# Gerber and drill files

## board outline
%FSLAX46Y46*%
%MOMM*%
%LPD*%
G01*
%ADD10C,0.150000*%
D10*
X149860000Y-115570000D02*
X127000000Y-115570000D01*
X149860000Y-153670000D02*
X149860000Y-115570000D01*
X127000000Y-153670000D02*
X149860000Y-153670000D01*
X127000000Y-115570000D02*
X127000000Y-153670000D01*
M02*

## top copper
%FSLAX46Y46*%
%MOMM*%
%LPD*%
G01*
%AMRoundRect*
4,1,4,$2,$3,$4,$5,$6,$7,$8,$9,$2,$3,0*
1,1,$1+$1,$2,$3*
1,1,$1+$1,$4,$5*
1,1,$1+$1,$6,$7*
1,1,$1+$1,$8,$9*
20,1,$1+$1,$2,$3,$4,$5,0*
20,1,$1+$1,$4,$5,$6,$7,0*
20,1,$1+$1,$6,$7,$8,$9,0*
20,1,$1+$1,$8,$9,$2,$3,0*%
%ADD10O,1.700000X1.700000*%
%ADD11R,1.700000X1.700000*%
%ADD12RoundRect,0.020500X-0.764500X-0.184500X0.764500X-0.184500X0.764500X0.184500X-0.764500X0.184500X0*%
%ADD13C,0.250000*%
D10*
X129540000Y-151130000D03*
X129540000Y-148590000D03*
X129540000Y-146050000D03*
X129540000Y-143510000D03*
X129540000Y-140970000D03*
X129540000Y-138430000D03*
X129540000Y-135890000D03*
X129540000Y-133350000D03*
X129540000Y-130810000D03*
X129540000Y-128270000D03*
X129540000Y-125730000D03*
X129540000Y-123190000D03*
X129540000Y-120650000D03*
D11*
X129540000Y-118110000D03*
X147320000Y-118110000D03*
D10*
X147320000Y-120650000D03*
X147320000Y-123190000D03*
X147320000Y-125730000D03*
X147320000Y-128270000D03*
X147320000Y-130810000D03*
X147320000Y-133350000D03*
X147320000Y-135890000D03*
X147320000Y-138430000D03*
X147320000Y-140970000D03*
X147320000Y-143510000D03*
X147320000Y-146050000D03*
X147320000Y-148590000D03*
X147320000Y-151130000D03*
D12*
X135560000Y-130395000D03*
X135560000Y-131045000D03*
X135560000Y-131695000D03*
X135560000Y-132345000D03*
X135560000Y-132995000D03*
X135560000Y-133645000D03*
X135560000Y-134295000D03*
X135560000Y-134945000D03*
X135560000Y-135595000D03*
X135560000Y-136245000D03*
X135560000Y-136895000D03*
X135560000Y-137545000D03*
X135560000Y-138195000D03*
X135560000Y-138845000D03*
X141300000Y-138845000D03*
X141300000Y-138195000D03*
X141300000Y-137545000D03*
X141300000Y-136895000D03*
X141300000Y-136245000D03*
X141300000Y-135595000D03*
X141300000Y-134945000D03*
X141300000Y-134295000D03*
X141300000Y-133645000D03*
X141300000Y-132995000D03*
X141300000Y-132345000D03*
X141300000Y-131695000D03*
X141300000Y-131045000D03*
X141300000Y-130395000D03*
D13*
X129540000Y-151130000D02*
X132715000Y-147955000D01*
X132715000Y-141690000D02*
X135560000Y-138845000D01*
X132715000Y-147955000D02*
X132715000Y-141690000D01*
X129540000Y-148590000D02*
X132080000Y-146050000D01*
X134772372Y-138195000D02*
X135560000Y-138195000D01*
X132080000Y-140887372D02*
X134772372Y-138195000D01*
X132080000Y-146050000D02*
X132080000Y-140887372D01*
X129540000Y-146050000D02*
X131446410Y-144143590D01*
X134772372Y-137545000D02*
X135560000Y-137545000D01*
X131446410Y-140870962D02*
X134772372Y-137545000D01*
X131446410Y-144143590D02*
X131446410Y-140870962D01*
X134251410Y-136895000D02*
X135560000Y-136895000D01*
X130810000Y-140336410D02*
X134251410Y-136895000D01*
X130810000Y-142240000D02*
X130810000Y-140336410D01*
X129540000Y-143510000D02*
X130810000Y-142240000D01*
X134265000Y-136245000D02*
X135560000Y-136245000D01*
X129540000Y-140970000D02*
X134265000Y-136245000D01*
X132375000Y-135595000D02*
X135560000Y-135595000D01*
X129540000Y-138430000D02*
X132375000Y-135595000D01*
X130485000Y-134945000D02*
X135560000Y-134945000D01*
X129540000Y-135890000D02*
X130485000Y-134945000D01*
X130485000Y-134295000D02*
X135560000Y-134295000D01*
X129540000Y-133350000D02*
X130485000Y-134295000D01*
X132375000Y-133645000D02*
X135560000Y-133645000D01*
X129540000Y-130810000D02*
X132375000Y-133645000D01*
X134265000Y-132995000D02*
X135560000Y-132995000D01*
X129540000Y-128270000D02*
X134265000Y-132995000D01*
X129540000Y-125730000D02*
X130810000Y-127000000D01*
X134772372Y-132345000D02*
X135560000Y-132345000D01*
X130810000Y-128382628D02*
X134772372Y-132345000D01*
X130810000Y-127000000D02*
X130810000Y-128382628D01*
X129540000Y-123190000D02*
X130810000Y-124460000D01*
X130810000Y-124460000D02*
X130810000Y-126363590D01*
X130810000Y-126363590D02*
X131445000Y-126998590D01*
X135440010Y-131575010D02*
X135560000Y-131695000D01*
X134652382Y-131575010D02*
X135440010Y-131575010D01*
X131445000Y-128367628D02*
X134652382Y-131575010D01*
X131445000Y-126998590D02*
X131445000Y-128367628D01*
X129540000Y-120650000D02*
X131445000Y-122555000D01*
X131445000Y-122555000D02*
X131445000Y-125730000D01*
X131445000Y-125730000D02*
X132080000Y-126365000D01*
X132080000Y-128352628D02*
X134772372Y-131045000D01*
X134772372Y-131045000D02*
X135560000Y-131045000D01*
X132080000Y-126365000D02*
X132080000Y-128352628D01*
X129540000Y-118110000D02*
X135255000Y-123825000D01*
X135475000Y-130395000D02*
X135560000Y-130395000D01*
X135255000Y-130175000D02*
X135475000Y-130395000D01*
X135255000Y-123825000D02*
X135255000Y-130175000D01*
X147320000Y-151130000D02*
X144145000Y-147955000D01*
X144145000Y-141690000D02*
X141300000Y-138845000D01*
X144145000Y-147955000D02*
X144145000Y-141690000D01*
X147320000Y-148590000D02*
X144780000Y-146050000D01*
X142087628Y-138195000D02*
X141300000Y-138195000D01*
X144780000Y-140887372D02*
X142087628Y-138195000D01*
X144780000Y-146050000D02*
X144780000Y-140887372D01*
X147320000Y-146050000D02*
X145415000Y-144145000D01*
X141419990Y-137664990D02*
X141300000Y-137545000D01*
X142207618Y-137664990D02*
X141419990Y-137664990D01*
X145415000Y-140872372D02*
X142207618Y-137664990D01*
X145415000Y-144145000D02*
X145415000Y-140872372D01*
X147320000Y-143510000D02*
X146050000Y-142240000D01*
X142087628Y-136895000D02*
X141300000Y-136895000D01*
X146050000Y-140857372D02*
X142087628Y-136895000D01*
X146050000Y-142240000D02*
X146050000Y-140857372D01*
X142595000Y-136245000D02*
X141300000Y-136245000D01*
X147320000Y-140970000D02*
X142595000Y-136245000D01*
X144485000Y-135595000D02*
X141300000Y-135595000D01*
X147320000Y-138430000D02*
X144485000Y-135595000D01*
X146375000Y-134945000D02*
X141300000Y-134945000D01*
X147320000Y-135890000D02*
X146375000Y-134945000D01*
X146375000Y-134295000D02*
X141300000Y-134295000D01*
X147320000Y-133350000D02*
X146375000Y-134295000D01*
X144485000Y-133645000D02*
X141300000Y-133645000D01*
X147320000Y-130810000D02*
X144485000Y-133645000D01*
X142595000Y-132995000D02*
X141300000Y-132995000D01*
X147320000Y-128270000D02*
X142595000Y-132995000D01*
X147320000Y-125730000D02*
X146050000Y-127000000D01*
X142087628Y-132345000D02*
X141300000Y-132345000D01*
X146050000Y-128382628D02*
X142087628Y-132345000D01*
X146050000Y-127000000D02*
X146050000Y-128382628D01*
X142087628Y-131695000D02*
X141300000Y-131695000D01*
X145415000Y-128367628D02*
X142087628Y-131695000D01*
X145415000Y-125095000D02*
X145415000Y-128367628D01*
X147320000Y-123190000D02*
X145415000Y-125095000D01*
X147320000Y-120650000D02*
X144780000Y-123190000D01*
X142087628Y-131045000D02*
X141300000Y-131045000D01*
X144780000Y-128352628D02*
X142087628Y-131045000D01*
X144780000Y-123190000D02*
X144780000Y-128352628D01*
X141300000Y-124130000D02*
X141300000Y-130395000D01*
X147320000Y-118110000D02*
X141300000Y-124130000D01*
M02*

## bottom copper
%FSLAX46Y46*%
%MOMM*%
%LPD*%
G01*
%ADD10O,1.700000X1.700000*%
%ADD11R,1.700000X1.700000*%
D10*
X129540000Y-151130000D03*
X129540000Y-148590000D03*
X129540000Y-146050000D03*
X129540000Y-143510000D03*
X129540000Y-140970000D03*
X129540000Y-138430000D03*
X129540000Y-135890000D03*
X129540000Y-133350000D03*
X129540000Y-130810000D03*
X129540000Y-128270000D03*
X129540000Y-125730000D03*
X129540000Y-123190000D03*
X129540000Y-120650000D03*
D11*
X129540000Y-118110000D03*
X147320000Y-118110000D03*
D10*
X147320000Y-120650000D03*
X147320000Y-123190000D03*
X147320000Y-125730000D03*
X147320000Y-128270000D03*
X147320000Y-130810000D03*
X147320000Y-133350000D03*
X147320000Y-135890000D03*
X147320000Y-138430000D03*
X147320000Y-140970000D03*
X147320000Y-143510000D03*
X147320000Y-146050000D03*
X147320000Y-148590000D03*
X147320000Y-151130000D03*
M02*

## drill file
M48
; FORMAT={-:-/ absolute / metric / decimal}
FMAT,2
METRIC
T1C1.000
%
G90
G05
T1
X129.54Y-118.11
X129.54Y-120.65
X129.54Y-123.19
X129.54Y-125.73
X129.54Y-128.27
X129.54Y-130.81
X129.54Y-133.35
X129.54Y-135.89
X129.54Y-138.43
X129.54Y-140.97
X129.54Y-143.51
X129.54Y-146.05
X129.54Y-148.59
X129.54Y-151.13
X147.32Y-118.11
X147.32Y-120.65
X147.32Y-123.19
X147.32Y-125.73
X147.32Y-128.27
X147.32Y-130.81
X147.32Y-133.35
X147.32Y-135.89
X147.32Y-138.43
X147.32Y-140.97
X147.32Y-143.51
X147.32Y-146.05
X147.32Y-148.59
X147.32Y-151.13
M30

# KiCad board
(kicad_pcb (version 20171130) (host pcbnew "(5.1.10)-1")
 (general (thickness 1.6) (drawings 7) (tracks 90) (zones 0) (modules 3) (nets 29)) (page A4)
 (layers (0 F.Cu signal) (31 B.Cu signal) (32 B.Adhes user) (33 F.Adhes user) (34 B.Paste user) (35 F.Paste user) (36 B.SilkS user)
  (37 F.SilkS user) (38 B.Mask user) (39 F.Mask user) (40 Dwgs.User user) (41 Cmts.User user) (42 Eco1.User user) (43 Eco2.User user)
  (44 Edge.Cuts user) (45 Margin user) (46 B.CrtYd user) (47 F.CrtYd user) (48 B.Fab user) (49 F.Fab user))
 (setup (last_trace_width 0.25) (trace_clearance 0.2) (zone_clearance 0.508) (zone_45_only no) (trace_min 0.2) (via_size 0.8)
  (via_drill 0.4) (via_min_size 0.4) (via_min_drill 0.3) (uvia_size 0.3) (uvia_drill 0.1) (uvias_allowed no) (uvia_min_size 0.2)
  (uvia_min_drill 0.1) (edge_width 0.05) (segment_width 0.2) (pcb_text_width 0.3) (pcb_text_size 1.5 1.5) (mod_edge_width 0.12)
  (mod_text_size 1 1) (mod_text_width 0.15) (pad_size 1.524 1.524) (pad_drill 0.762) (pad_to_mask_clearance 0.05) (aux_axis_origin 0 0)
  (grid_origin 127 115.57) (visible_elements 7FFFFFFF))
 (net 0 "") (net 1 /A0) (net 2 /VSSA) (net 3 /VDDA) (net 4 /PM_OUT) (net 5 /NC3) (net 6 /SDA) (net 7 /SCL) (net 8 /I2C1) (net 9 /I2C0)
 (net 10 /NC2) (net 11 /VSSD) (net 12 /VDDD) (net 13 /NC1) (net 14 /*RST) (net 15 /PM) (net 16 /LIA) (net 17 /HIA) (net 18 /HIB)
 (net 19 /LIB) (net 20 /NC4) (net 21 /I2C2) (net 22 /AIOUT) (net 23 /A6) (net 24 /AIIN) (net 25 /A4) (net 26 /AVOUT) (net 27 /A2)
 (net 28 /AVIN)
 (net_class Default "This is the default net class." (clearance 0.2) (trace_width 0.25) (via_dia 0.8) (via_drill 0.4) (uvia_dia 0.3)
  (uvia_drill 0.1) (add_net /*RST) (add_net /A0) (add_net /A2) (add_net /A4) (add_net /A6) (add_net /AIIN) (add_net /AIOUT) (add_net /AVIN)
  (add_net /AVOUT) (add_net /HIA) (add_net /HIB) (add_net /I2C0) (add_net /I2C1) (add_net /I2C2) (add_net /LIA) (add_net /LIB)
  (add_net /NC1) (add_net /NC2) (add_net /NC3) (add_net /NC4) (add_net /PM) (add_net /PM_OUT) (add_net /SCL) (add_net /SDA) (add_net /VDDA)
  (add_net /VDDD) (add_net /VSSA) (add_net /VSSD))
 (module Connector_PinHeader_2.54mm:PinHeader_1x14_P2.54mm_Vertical (layer F.Cu) (at 129.54 118.11)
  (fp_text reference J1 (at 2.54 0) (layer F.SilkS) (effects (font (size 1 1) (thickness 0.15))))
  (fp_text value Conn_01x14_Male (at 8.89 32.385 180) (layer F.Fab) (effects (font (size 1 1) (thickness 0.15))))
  (pad 14 thru_hole oval (at 0 33.02) (size 1.7 1.7) (drill 1) (layers *.Cu *.Mask) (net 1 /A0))
  (pad 13 thru_hole oval (at 0 30.48) (size 1.7 1.7) (drill 1) (layers *.Cu *.Mask) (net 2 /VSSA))
  (pad 12 thru_hole oval (at 0 27.94) (size 1.7 1.7) (drill 1) (layers *.Cu *.Mask) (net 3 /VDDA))
  (pad 11 thru_hole oval (at 0 25.4) (size 1.7 1.7) (drill 1) (layers *.Cu *.Mask) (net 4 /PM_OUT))
  (pad 10 thru_hole oval (at 0 22.86) (size 1.7 1.7) (drill 1) (layers *.Cu *.Mask) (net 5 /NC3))
  (pad 9 thru_hole oval (at 0 20.32) (size 1.7 1.7) (drill 1) (layers *.Cu *.Mask) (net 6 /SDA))
  (pad 8 thru_hole oval (at 0 17.78) (size 1.7 1.7) (drill 1) (layers *.Cu *.Mask) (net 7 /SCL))
  (pad 7 thru_hole oval (at 0 15.24) (size 1.7 1.7) (drill 1) (layers *.Cu *.Mask) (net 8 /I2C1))
  (pad 6 thru_hole oval (at 0 12.7) (size 1.7 1.7) (drill 1) (layers *.Cu *.Mask) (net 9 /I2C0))
  (pad 5 thru_hole oval (at 0 10.16) (size 1.7 1.7) (drill 1) (layers *.Cu *.Mask) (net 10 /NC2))
  (pad 4 thru_hole oval (at 0 7.62) (size 1.7 1.7) (drill 1) (layers *.Cu *.Mask) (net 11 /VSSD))
  (pad 3 thru_hole oval (at 0 5.08) (size 1.7 1.7) (drill 1) (layers *.Cu *.Mask) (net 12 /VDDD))
  (pad 2 thru_hole oval (at 0 2.54) (size 1.7 1.7) (drill 1) (layers *.Cu *.Mask) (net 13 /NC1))
  (pad 1 thru_hole rect (at 0 0) (size 1.7 1.7) (drill 1) (layers *.Cu *.Mask) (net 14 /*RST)))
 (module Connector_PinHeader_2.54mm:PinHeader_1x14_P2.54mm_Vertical (layer F.Cu) (at 147.32 118.11)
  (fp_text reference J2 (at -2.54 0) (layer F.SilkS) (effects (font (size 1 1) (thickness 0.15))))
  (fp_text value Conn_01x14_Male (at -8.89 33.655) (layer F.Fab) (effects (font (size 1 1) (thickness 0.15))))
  (pad 1 thru_hole rect (at 0 0) (size 1.7 1.7) (drill 1) (layers *.Cu *.Mask) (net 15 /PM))
  (pad 2 thru_hole oval (at 0 2.54) (size 1.7 1.7) (drill 1) (layers *.Cu *.Mask) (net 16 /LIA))
  (pad 3 thru_hole oval (at 0 5.08) (size 1.7 1.7) (drill 1) (layers *.Cu *.Mask) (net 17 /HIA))
  (pad 4 thru_hole oval (at 0 7.62) (size 1.7 1.7) (drill 1) (layers *.Cu *.Mask) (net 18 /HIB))
  (pad 5 thru_hole oval (at 0 10.16) (size 1.7 1.7) (drill 1) (layers *.Cu *.Mask) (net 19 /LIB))
  (pad 6 thru_hole oval (at 0 12.7) (size 1.7 1.7) (drill 1) (layers *.Cu *.Mask) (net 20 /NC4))
  (pad 7 thru_hole oval (at 0 15.24) (size 1.7 1.7) (drill 1) (layers *.Cu *.Mask) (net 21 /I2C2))
  (pad 8 thru_hole oval (at 0 17.78) (size 1.7 1.7) (drill 1) (layers *.Cu *.Mask) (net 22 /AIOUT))
  (pad 9 thru_hole oval (at 0 20.32) (size 1.7 1.7) (drill 1) (layers *.Cu *.Mask) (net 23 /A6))
  (pad 10 thru_hole oval (at 0 22.86) (size 1.7 1.7) (drill 1) (layers *.Cu *.Mask) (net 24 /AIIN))
  (pad 11 thru_hole oval (at 0 25.4) (size 1.7 1.7) (drill 1) (layers *.Cu *.Mask) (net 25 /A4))
  (pad 12 thru_hole oval (at 0 27.94) (size 1.7 1.7) (drill 1) (layers *.Cu *.Mask) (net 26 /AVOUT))
  (pad 13 thru_hole oval (at 0 30.48) (size 1.7 1.7) (drill 1) (layers *.Cu *.Mask) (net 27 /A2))
  (pad 14 thru_hole oval (at 0 33.02) (size 1.7 1.7) (drill 1) (layers *.Cu *.Mask) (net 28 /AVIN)))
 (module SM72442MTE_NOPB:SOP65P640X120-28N (layer F.Cu) (at 138.43 134.62)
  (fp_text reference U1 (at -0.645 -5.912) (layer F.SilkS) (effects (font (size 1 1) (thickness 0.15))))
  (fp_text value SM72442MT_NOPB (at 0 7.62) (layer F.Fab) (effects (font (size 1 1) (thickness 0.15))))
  (pad 1 smd roundrect (at -2.87 -4.225) (size 1.57 0.41) (layers F.Cu F.Paste F.Mask) (roundrect_rratio 0.05) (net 14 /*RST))
  (pad 2 smd roundrect (at -2.87 -3.575) (size 1.57 0.41) (layers F.Cu F.Paste F.Mask) (roundrect_rratio 0.05) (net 13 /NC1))
  (pad 3 smd roundrect (at -2.87 -2.925) (size 1.57 0.41) (layers F.Cu F.Paste F.Mask) (roundrect_rratio 0.05) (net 12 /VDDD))
  (pad 4 smd roundrect (at -2.87 -2.275) (size 1.57 0.41) (layers F.Cu F.Paste F.Mask) (roundrect_rratio 0.05) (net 11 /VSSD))
  (pad 5 smd roundrect (at -2.87 -1.625) (size 1.57 0.41) (layers F.Cu F.Paste F.Mask) (roundrect_rratio 0.05) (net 10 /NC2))
  (pad 6 smd roundrect (at -2.87 -0.975) (size 1.57 0.41) (layers F.Cu F.Paste F.Mask) (roundrect_rratio 0.05) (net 9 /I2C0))
  (pad 7 smd roundrect (at -2.87 -0.325) (size 1.57 0.41) (layers F.Cu F.Paste F.Mask) (roundrect_rratio 0.05) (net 8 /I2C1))
  (pad 8 smd roundrect (at -2.87 0.325) (size 1.57 0.41) (layers F.Cu F.Paste F.Mask) (roundrect_rratio 0.05) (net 7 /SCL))
  (pad 9 smd roundrect (at -2.87 0.975) (size 1.57 0.41) (layers F.Cu F.Paste F.Mask) (roundrect_rratio 0.05) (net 6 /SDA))
  (pad 10 smd roundrect (at -2.87 1.625) (size 1.57 0.41) (layers F.Cu F.Paste F.Mask) (roundrect_rratio 0.05) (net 5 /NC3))
  (pad 11 smd roundrect (at -2.87 2.275) (size 1.57 0.41) (layers F.Cu F.Paste F.Mask) (roundrect_rratio 0.05) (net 4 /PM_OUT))
  (pad 12 smd roundrect (at -2.87 2.925) (size 1.57 0.41) (layers F.Cu F.Paste F.Mask) (roundrect_rratio 0.05) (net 3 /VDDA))
  (pad 13 smd roundrect (at -2.87 3.575) (size 1.57 0.41) (layers F.Cu F.Paste F.Mask) (roundrect_rratio 0.05) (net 2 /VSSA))
  (pad 14 smd roundrect (at -2.87 4.225) (size 1.57 0.41) (layers F.Cu F.Paste F.Mask) (roundrect_rratio 0.05) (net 1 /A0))
  (pad 15 smd roundrect (at 2.87 4.225) (size 1.57 0.41) (layers F.Cu F.Paste F.Mask) (roundrect_rratio 0.05) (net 28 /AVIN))
  (pad 16 smd roundrect (at 2.87 3.575) (size 1.57 0.41) (layers F.Cu F.Paste F.Mask) (roundrect_rratio 0.05) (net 27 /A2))
  (pad 17 smd roundrect (at 2.87 2.925) (size 1.57 0.41) (layers F.Cu F.Paste F.Mask) (roundrect_rratio 0.05) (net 26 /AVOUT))
  (pad 18 smd roundrect (at 2.87 2.275) (size 1.57 0.41) (layers F.Cu F.Paste F.Mask) (roundrect_rratio 0.05) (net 25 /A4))
  (pad 19 smd roundrect (at 2.87 1.625) (size 1.57 0.41) (layers F.Cu F.Paste F.Mask) (roundrect_rratio 0.05) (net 24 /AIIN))
  (pad 20 smd roundrect (at 2.87 0.975) (size 1.57 0.41) (layers F.Cu F.Paste F.Mask) (roundrect_rratio 0.05) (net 23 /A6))
  (pad 21 smd roundrect (at 2.87 0.325) (size 1.57 0.41) (layers F.Cu F.Paste F.Mask) (roundrect_rratio 0.05) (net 22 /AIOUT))
  (pad 22 smd roundrect (at 2.87 -0.325) (size 1.57 0.41) (layers F.Cu F.Paste F.Mask) (roundrect_rratio 0.05) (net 21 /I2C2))
  (pad 23 smd roundrect (at 2.87 -0.975) (size 1.57 0.41) (layers F.Cu F.Paste F.Mask) (roundrect_rratio 0.05) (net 20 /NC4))
  (pad 24 smd roundrect (at 2.87 -1.625) (size 1.57 0.41) (layers F.Cu F.Paste F.Mask) (roundrect_rratio 0.05) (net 19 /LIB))
  (pad 25 smd roundrect (at 2.87 -2.275) (size 1.57 0.41) (layers F.Cu F.Paste F.Mask) (roundrect_rratio 0.05) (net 18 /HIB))
  (pad 26 smd roundrect (at 2.87 -2.925) (size 1.57 0.41) (layers F.Cu F.Paste F.Mask) (roundrect_rratio 0.05) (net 17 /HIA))
  (pad 27 smd roundrect (at 2.87 -3.575) (size 1.57 0.41) (layers F.Cu F.Paste F.Mask) (roundrect_rratio 0.05) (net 16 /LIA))
  (pad 28 smd roundrect (at 2.87 -4.225) (size 1.57 0.41) (layers F.Cu F.Paste F.Mask) (roundrect_rratio 0.05) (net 15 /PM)))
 (gr_line (start 149.86 115.57) (end 127 115.57) (layer Edge.Cuts) (width 0.15))
 (gr_line (start 149.86 153.67) (end 149.86 115.57) (layer Edge.Cuts) (width 0.15))
 (gr_line (start 127 153.67) (end 149.86 153.67) (layer Edge.Cuts) (width 0.15))
 (gr_line (start 127 115.57) (end 127 153.67) (layer Edge.Cuts) (width 0.15))
 (segment (start 129.54 151.13) (end 132.715 147.955) (width 0.25) (layer F.Cu) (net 1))
 (segment (start 132.715 141.69) (end 135.56 138.845) (width 0.25) (layer F.Cu) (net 1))
 (segment (start 132.715 147.955) (end 132.715 141.69) (width 0.25) (layer F.Cu) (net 1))
 (segment (start 129.54 148.59) (end 132.08 146.05) (width 0.25) (layer F.Cu) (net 2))
 (segment (start 134.772372 138.195) (end 135.56 138.195) (width 0.25) (layer F.Cu) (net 2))
 (segment (start 132.08 140.887372) (end 134.772372 138.195) (width 0.25) (layer F.Cu) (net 2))
 (segment (start 132.08 146.05) (end 132.08 140.887372) (width 0.25) (layer F.Cu) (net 2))
 (segment (start 129.54 146.05) (end 131.44641 144.14359) (width 0.25) (layer F.Cu) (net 3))
 (segment (start 134.772372 137.545) (end 135.56 137.545) (width 0.25) (layer F.Cu) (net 3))
 (segment (start 131.44641 140.870962) (end 134.772372 137.545) (width 0.25) (layer F.Cu) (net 3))
 (segment (start 131.44641 144.14359) (end 131.44641 140.870962) (width 0.25) (layer F.Cu) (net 3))
 (segment (start 134.25141 136.895) (end 135.56 136.895) (width 0.25) (layer F.Cu) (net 4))
 (segment (start 130.81 140.33641) (end 134.25141 136.895) (width 0.25) (layer F.Cu) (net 4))
 (segment (start 130.81 142.24) (end 130.81 140.33641) (width 0.25) (layer F.Cu) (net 4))
 (segment (start 129.54 143.51) (end 130.81 142.24) (width 0.25) (layer F.Cu) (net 4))
 (segment (start 134.265 136.245) (end 135.56 136.245) (width 0.25) (layer F.Cu) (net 5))
 (segment (start 129.54 140.97) (end 134.265 136.245) (width 0.25) (layer F.Cu) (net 5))
 (segment (start 132.375 135.595) (end 135.56 135.595) (width 0.25) (layer F.Cu) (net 6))
 (segment (start 129.54 138.43) (end 132.375 135.595) (width 0.25) (layer F.Cu) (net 6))
 (segment (start 130.485 134.945) (end 135.56 134.945) (width 0.25) (layer F.Cu) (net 7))
 (segment (start 129.54 135.89) (end 130.485 134.945) (width 0.25) (layer F.Cu) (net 7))
 (segment (start 130.485 134.295) (end 135.56 134.295) (width 0.25) (layer F.Cu) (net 8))
 (segment (start 129.54 133.35) (end 130.485 134.295) (width 0.25) (layer F.Cu) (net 8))
 (segment (start 132.375 133.645) (end 135.56 133.645) (width 0.25) (layer F.Cu) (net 9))
 (segment (start 129.54 130.81) (end 132.375 133.645) (width 0.25) (layer F.Cu) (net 9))
 (segment (start 134.265 132.995) (end 135.56 132.995) (width 0.25) (layer F.Cu) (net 10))
 (segment (start 129.54 128.27) (end 134.265 132.995) (width 0.25) (layer F.Cu) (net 10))
 (segment (start 129.54 125.73) (end 130.81 127) (width 0.25) (layer F.Cu) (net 11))
 (segment (start 134.772372 132.345) (end 135.56 132.345) (width 0.25) (layer F.Cu) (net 11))
 (segment (start 130.81 128.382628) (end 134.772372 132.345) (width 0.25) (layer F.Cu) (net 11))
 (segment (start 130.81 127) (end 130.81 128.382628) (width 0.25) (layer F.Cu) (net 11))
 (segment (start 129.54 123.19) (end 130.81 124.46) (width 0.25) (layer F.Cu) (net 12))
 (segment (start 130.81 124.46) (end 130.81 126.36359) (width 0.25) (layer F.Cu) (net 12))
 (segment (start 130.81 126.36359) (end 131.445 126.99859) (width 0.25) (layer F.Cu) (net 12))
 (segment (start 135.44001 131.57501) (end 135.56 131.695) (width 0.25) (layer F.Cu) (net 12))
 (segment (start 134.652382 131.57501) (end 135.44001 131.57501) (width 0.25) (layer F.Cu) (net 12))
 (segment (start 131.445 128.367628) (end 134.652382 131.57501) (width 0.25) (layer F.Cu) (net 12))
 (segment (start 131.445 126.99859) (end 131.445 128.367628) (width 0.25) (layer F.Cu) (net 12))
 (segment (start 129.54 120.65) (end 131.445 122.555) (width 0.25) (layer F.Cu) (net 13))
 (segment (start 131.445 122.555) (end 131.445 125.73) (width 0.25) (layer F.Cu) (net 13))
 (segment (start 131.445 125.73) (end 132.08 126.365) (width 0.25) (layer F.Cu) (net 13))
 (segment (start 132.08 128.352628) (end 134.772372 131.045) (width 0.25) (layer F.Cu) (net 13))
 (segment (start 134.772372 131.045) (end 135.56 131.045) (width 0.25) (layer F.Cu) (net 13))
 (segment (start 132.08 126.365) (end 132.08 128.352628) (width 0.25) (layer F.Cu) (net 13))
 (segment (start 129.54 118.11) (end 135.255 123.825) (width 0.25) (layer F.Cu) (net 14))
 (segment (start 135.475 130.395) (end 135.56 130.395) (width 0.25) (layer F.Cu) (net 14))
 (segment (start 135.255 130.175) (end 135.475 130.395) (width 0.25) (layer F.Cu) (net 14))
 (segment (start 135.255 123.825) (end 135.255 130.175) (width 0.25) (layer F.Cu) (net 14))
 (segment (start 147.32 151.13) (end 144.145 147.955) (width 0.25) (layer F.Cu) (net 28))
 (segment (start 144.145 141.69) (end 141.3 138.845) (width 0.25) (layer F.Cu) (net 28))
 (segment (start 144.145 147.955) (end 144.145 141.69) (width 0.25) (layer F.Cu) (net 28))
 (segment (start 147.32 148.59) (end 144.78 146.05) (width 0.25) (layer F.Cu) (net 27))
 (segment (start 142.087628 138.195) (end 141.3 138.195) (width 0.25) (layer F.Cu) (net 27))
 (segment (start 144.78 140.887372) (end 142.087628 138.195) (width 0.25) (layer F.Cu) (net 27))
 (segment (start 144.78 146.05) (end 144.78 140.887372) (width 0.25) (layer F.Cu) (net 27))
 (segment (start 147.32 146.05) (end 145.415 144.145) (width 0.25) (layer F.Cu) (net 26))
 (segment (start 141.41999 137.66499) (end 141.3 137.545) (width 0.25) (layer F.Cu) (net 26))
 (segment (start 142.207618 137.66499) (end 141.41999 137.66499) (width 0.25) (layer F.Cu) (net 26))
 (segment (start 145.415 140.872372) (end 142.207618 137.66499) (width 0.25) (layer F.Cu) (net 26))
 (segment (start 145.415 144.145) (end 145.415 140.872372) (width 0.25) (layer F.Cu) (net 26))
 (segment (start 147.32 143.51) (end 146.05 142.24) (width 0.25) (layer F.Cu) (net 25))
 (segment (start 142.087628 136.895) (end 141.3 136.895) (width 0.25) (layer F.Cu) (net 25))
 (segment (start 146.05 140.857372) (end 142.087628 136.895) (width 0.25) (layer F.Cu) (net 25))
 (segment (start 146.05 142.24) (end 146.05 140.857372) (width 0.25) (layer F.Cu) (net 25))
 (segment (start 142.595 136.245) (end 141.3 136.245) (width 0.25) (layer F.Cu) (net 24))
 (segment (start 147.32 140.97) (end 142.595 136.245) (width 0.25) (layer F.Cu) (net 24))
 (segment (start 144.485 135.595) (end 141.3 135.595) (width 0.25) (layer F.Cu) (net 23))
 (segment (start 147.32 138.43) (end 144.485 135.595) (width 0.25) (layer F.Cu) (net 23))
 (segment (start 146.375 134.945) (end 141.3 134.945) (width 0.25) (layer F.Cu) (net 22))
 (segment (start 147.32 135.89) (end 146.375 134.945) (width 0.25) (layer F.Cu) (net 22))
 (segment (start 146.375 134.295) (end 141.3 134.295) (width 0.25) (layer F.Cu) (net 21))
 (segment (start 147.32 133.35) (end 146.375 134.295) (width 0.25) (layer F.Cu) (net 21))
 (segment (start 144.485 133.645) (end 141.3 133.645) (width 0.25) (layer F.Cu) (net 20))
 (segment (start 147.32 130.81) (end 144.485 133.645) (width 0.25) (layer F.Cu) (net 20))
 (segment (start 142.595 132.995) (end 141.3 132.995) (width 0.25) (layer F.Cu) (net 19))
 (segment (start 147.32 128.27) (end 142.595 132.995) (width 0.25) (layer F.Cu) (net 19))
 (segment (start 147.32 125.73) (end 146.05 127) (width 0.25) (layer F.Cu) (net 18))
 (segment (start 142.087628 132.345) (end 141.3 132.345) (width 0.25) (layer F.Cu) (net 18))
 (segment (start 146.05 128.382628) (end 142.087628 132.345) (width 0.25) (layer F.Cu) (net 18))
 (segment (start 146.05 127) (end 146.05 128.382628) (width 0.25) (layer F.Cu) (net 18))
 (segment (start 142.087628 131.695) (end 141.3 131.695) (width 0.25) (layer F.Cu) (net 17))
 (segment (start 145.415 128.367628) (end 142.087628 131.695) (width 0.25) (layer F.Cu) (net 17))
 (segment (start 145.415 125.095) (end 145.415 128.367628) (width 0.25) (layer F.Cu) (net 17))
 (segment (start 147.32 123.19) (end 145.415 125.095) (width 0.25) (layer F.Cu) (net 17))
 (segment (start 147.32 120.65) (end 144.78 123.19) (width 0.25) (layer F.Cu) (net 16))
 (segment (start 142.087628 131.045) (end 141.3 131.045) (width 0.25) (layer F.Cu) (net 16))
 (segment (start 144.78 128.352628) (end 142.087628 131.045) (width 0.25) (layer F.Cu) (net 16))
 (segment (start 144.78 123.19) (end 144.78 128.352628) (width 0.25) (layer F.Cu) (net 16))
 (segment (start 141.3 124.13) (end 141.3 130.395) (width 0.25) (layer F.Cu) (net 15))
 (segment (start 147.32 118.11) (end 141.3 124.13) (width 0.25) (layer F.Cu) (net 15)))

